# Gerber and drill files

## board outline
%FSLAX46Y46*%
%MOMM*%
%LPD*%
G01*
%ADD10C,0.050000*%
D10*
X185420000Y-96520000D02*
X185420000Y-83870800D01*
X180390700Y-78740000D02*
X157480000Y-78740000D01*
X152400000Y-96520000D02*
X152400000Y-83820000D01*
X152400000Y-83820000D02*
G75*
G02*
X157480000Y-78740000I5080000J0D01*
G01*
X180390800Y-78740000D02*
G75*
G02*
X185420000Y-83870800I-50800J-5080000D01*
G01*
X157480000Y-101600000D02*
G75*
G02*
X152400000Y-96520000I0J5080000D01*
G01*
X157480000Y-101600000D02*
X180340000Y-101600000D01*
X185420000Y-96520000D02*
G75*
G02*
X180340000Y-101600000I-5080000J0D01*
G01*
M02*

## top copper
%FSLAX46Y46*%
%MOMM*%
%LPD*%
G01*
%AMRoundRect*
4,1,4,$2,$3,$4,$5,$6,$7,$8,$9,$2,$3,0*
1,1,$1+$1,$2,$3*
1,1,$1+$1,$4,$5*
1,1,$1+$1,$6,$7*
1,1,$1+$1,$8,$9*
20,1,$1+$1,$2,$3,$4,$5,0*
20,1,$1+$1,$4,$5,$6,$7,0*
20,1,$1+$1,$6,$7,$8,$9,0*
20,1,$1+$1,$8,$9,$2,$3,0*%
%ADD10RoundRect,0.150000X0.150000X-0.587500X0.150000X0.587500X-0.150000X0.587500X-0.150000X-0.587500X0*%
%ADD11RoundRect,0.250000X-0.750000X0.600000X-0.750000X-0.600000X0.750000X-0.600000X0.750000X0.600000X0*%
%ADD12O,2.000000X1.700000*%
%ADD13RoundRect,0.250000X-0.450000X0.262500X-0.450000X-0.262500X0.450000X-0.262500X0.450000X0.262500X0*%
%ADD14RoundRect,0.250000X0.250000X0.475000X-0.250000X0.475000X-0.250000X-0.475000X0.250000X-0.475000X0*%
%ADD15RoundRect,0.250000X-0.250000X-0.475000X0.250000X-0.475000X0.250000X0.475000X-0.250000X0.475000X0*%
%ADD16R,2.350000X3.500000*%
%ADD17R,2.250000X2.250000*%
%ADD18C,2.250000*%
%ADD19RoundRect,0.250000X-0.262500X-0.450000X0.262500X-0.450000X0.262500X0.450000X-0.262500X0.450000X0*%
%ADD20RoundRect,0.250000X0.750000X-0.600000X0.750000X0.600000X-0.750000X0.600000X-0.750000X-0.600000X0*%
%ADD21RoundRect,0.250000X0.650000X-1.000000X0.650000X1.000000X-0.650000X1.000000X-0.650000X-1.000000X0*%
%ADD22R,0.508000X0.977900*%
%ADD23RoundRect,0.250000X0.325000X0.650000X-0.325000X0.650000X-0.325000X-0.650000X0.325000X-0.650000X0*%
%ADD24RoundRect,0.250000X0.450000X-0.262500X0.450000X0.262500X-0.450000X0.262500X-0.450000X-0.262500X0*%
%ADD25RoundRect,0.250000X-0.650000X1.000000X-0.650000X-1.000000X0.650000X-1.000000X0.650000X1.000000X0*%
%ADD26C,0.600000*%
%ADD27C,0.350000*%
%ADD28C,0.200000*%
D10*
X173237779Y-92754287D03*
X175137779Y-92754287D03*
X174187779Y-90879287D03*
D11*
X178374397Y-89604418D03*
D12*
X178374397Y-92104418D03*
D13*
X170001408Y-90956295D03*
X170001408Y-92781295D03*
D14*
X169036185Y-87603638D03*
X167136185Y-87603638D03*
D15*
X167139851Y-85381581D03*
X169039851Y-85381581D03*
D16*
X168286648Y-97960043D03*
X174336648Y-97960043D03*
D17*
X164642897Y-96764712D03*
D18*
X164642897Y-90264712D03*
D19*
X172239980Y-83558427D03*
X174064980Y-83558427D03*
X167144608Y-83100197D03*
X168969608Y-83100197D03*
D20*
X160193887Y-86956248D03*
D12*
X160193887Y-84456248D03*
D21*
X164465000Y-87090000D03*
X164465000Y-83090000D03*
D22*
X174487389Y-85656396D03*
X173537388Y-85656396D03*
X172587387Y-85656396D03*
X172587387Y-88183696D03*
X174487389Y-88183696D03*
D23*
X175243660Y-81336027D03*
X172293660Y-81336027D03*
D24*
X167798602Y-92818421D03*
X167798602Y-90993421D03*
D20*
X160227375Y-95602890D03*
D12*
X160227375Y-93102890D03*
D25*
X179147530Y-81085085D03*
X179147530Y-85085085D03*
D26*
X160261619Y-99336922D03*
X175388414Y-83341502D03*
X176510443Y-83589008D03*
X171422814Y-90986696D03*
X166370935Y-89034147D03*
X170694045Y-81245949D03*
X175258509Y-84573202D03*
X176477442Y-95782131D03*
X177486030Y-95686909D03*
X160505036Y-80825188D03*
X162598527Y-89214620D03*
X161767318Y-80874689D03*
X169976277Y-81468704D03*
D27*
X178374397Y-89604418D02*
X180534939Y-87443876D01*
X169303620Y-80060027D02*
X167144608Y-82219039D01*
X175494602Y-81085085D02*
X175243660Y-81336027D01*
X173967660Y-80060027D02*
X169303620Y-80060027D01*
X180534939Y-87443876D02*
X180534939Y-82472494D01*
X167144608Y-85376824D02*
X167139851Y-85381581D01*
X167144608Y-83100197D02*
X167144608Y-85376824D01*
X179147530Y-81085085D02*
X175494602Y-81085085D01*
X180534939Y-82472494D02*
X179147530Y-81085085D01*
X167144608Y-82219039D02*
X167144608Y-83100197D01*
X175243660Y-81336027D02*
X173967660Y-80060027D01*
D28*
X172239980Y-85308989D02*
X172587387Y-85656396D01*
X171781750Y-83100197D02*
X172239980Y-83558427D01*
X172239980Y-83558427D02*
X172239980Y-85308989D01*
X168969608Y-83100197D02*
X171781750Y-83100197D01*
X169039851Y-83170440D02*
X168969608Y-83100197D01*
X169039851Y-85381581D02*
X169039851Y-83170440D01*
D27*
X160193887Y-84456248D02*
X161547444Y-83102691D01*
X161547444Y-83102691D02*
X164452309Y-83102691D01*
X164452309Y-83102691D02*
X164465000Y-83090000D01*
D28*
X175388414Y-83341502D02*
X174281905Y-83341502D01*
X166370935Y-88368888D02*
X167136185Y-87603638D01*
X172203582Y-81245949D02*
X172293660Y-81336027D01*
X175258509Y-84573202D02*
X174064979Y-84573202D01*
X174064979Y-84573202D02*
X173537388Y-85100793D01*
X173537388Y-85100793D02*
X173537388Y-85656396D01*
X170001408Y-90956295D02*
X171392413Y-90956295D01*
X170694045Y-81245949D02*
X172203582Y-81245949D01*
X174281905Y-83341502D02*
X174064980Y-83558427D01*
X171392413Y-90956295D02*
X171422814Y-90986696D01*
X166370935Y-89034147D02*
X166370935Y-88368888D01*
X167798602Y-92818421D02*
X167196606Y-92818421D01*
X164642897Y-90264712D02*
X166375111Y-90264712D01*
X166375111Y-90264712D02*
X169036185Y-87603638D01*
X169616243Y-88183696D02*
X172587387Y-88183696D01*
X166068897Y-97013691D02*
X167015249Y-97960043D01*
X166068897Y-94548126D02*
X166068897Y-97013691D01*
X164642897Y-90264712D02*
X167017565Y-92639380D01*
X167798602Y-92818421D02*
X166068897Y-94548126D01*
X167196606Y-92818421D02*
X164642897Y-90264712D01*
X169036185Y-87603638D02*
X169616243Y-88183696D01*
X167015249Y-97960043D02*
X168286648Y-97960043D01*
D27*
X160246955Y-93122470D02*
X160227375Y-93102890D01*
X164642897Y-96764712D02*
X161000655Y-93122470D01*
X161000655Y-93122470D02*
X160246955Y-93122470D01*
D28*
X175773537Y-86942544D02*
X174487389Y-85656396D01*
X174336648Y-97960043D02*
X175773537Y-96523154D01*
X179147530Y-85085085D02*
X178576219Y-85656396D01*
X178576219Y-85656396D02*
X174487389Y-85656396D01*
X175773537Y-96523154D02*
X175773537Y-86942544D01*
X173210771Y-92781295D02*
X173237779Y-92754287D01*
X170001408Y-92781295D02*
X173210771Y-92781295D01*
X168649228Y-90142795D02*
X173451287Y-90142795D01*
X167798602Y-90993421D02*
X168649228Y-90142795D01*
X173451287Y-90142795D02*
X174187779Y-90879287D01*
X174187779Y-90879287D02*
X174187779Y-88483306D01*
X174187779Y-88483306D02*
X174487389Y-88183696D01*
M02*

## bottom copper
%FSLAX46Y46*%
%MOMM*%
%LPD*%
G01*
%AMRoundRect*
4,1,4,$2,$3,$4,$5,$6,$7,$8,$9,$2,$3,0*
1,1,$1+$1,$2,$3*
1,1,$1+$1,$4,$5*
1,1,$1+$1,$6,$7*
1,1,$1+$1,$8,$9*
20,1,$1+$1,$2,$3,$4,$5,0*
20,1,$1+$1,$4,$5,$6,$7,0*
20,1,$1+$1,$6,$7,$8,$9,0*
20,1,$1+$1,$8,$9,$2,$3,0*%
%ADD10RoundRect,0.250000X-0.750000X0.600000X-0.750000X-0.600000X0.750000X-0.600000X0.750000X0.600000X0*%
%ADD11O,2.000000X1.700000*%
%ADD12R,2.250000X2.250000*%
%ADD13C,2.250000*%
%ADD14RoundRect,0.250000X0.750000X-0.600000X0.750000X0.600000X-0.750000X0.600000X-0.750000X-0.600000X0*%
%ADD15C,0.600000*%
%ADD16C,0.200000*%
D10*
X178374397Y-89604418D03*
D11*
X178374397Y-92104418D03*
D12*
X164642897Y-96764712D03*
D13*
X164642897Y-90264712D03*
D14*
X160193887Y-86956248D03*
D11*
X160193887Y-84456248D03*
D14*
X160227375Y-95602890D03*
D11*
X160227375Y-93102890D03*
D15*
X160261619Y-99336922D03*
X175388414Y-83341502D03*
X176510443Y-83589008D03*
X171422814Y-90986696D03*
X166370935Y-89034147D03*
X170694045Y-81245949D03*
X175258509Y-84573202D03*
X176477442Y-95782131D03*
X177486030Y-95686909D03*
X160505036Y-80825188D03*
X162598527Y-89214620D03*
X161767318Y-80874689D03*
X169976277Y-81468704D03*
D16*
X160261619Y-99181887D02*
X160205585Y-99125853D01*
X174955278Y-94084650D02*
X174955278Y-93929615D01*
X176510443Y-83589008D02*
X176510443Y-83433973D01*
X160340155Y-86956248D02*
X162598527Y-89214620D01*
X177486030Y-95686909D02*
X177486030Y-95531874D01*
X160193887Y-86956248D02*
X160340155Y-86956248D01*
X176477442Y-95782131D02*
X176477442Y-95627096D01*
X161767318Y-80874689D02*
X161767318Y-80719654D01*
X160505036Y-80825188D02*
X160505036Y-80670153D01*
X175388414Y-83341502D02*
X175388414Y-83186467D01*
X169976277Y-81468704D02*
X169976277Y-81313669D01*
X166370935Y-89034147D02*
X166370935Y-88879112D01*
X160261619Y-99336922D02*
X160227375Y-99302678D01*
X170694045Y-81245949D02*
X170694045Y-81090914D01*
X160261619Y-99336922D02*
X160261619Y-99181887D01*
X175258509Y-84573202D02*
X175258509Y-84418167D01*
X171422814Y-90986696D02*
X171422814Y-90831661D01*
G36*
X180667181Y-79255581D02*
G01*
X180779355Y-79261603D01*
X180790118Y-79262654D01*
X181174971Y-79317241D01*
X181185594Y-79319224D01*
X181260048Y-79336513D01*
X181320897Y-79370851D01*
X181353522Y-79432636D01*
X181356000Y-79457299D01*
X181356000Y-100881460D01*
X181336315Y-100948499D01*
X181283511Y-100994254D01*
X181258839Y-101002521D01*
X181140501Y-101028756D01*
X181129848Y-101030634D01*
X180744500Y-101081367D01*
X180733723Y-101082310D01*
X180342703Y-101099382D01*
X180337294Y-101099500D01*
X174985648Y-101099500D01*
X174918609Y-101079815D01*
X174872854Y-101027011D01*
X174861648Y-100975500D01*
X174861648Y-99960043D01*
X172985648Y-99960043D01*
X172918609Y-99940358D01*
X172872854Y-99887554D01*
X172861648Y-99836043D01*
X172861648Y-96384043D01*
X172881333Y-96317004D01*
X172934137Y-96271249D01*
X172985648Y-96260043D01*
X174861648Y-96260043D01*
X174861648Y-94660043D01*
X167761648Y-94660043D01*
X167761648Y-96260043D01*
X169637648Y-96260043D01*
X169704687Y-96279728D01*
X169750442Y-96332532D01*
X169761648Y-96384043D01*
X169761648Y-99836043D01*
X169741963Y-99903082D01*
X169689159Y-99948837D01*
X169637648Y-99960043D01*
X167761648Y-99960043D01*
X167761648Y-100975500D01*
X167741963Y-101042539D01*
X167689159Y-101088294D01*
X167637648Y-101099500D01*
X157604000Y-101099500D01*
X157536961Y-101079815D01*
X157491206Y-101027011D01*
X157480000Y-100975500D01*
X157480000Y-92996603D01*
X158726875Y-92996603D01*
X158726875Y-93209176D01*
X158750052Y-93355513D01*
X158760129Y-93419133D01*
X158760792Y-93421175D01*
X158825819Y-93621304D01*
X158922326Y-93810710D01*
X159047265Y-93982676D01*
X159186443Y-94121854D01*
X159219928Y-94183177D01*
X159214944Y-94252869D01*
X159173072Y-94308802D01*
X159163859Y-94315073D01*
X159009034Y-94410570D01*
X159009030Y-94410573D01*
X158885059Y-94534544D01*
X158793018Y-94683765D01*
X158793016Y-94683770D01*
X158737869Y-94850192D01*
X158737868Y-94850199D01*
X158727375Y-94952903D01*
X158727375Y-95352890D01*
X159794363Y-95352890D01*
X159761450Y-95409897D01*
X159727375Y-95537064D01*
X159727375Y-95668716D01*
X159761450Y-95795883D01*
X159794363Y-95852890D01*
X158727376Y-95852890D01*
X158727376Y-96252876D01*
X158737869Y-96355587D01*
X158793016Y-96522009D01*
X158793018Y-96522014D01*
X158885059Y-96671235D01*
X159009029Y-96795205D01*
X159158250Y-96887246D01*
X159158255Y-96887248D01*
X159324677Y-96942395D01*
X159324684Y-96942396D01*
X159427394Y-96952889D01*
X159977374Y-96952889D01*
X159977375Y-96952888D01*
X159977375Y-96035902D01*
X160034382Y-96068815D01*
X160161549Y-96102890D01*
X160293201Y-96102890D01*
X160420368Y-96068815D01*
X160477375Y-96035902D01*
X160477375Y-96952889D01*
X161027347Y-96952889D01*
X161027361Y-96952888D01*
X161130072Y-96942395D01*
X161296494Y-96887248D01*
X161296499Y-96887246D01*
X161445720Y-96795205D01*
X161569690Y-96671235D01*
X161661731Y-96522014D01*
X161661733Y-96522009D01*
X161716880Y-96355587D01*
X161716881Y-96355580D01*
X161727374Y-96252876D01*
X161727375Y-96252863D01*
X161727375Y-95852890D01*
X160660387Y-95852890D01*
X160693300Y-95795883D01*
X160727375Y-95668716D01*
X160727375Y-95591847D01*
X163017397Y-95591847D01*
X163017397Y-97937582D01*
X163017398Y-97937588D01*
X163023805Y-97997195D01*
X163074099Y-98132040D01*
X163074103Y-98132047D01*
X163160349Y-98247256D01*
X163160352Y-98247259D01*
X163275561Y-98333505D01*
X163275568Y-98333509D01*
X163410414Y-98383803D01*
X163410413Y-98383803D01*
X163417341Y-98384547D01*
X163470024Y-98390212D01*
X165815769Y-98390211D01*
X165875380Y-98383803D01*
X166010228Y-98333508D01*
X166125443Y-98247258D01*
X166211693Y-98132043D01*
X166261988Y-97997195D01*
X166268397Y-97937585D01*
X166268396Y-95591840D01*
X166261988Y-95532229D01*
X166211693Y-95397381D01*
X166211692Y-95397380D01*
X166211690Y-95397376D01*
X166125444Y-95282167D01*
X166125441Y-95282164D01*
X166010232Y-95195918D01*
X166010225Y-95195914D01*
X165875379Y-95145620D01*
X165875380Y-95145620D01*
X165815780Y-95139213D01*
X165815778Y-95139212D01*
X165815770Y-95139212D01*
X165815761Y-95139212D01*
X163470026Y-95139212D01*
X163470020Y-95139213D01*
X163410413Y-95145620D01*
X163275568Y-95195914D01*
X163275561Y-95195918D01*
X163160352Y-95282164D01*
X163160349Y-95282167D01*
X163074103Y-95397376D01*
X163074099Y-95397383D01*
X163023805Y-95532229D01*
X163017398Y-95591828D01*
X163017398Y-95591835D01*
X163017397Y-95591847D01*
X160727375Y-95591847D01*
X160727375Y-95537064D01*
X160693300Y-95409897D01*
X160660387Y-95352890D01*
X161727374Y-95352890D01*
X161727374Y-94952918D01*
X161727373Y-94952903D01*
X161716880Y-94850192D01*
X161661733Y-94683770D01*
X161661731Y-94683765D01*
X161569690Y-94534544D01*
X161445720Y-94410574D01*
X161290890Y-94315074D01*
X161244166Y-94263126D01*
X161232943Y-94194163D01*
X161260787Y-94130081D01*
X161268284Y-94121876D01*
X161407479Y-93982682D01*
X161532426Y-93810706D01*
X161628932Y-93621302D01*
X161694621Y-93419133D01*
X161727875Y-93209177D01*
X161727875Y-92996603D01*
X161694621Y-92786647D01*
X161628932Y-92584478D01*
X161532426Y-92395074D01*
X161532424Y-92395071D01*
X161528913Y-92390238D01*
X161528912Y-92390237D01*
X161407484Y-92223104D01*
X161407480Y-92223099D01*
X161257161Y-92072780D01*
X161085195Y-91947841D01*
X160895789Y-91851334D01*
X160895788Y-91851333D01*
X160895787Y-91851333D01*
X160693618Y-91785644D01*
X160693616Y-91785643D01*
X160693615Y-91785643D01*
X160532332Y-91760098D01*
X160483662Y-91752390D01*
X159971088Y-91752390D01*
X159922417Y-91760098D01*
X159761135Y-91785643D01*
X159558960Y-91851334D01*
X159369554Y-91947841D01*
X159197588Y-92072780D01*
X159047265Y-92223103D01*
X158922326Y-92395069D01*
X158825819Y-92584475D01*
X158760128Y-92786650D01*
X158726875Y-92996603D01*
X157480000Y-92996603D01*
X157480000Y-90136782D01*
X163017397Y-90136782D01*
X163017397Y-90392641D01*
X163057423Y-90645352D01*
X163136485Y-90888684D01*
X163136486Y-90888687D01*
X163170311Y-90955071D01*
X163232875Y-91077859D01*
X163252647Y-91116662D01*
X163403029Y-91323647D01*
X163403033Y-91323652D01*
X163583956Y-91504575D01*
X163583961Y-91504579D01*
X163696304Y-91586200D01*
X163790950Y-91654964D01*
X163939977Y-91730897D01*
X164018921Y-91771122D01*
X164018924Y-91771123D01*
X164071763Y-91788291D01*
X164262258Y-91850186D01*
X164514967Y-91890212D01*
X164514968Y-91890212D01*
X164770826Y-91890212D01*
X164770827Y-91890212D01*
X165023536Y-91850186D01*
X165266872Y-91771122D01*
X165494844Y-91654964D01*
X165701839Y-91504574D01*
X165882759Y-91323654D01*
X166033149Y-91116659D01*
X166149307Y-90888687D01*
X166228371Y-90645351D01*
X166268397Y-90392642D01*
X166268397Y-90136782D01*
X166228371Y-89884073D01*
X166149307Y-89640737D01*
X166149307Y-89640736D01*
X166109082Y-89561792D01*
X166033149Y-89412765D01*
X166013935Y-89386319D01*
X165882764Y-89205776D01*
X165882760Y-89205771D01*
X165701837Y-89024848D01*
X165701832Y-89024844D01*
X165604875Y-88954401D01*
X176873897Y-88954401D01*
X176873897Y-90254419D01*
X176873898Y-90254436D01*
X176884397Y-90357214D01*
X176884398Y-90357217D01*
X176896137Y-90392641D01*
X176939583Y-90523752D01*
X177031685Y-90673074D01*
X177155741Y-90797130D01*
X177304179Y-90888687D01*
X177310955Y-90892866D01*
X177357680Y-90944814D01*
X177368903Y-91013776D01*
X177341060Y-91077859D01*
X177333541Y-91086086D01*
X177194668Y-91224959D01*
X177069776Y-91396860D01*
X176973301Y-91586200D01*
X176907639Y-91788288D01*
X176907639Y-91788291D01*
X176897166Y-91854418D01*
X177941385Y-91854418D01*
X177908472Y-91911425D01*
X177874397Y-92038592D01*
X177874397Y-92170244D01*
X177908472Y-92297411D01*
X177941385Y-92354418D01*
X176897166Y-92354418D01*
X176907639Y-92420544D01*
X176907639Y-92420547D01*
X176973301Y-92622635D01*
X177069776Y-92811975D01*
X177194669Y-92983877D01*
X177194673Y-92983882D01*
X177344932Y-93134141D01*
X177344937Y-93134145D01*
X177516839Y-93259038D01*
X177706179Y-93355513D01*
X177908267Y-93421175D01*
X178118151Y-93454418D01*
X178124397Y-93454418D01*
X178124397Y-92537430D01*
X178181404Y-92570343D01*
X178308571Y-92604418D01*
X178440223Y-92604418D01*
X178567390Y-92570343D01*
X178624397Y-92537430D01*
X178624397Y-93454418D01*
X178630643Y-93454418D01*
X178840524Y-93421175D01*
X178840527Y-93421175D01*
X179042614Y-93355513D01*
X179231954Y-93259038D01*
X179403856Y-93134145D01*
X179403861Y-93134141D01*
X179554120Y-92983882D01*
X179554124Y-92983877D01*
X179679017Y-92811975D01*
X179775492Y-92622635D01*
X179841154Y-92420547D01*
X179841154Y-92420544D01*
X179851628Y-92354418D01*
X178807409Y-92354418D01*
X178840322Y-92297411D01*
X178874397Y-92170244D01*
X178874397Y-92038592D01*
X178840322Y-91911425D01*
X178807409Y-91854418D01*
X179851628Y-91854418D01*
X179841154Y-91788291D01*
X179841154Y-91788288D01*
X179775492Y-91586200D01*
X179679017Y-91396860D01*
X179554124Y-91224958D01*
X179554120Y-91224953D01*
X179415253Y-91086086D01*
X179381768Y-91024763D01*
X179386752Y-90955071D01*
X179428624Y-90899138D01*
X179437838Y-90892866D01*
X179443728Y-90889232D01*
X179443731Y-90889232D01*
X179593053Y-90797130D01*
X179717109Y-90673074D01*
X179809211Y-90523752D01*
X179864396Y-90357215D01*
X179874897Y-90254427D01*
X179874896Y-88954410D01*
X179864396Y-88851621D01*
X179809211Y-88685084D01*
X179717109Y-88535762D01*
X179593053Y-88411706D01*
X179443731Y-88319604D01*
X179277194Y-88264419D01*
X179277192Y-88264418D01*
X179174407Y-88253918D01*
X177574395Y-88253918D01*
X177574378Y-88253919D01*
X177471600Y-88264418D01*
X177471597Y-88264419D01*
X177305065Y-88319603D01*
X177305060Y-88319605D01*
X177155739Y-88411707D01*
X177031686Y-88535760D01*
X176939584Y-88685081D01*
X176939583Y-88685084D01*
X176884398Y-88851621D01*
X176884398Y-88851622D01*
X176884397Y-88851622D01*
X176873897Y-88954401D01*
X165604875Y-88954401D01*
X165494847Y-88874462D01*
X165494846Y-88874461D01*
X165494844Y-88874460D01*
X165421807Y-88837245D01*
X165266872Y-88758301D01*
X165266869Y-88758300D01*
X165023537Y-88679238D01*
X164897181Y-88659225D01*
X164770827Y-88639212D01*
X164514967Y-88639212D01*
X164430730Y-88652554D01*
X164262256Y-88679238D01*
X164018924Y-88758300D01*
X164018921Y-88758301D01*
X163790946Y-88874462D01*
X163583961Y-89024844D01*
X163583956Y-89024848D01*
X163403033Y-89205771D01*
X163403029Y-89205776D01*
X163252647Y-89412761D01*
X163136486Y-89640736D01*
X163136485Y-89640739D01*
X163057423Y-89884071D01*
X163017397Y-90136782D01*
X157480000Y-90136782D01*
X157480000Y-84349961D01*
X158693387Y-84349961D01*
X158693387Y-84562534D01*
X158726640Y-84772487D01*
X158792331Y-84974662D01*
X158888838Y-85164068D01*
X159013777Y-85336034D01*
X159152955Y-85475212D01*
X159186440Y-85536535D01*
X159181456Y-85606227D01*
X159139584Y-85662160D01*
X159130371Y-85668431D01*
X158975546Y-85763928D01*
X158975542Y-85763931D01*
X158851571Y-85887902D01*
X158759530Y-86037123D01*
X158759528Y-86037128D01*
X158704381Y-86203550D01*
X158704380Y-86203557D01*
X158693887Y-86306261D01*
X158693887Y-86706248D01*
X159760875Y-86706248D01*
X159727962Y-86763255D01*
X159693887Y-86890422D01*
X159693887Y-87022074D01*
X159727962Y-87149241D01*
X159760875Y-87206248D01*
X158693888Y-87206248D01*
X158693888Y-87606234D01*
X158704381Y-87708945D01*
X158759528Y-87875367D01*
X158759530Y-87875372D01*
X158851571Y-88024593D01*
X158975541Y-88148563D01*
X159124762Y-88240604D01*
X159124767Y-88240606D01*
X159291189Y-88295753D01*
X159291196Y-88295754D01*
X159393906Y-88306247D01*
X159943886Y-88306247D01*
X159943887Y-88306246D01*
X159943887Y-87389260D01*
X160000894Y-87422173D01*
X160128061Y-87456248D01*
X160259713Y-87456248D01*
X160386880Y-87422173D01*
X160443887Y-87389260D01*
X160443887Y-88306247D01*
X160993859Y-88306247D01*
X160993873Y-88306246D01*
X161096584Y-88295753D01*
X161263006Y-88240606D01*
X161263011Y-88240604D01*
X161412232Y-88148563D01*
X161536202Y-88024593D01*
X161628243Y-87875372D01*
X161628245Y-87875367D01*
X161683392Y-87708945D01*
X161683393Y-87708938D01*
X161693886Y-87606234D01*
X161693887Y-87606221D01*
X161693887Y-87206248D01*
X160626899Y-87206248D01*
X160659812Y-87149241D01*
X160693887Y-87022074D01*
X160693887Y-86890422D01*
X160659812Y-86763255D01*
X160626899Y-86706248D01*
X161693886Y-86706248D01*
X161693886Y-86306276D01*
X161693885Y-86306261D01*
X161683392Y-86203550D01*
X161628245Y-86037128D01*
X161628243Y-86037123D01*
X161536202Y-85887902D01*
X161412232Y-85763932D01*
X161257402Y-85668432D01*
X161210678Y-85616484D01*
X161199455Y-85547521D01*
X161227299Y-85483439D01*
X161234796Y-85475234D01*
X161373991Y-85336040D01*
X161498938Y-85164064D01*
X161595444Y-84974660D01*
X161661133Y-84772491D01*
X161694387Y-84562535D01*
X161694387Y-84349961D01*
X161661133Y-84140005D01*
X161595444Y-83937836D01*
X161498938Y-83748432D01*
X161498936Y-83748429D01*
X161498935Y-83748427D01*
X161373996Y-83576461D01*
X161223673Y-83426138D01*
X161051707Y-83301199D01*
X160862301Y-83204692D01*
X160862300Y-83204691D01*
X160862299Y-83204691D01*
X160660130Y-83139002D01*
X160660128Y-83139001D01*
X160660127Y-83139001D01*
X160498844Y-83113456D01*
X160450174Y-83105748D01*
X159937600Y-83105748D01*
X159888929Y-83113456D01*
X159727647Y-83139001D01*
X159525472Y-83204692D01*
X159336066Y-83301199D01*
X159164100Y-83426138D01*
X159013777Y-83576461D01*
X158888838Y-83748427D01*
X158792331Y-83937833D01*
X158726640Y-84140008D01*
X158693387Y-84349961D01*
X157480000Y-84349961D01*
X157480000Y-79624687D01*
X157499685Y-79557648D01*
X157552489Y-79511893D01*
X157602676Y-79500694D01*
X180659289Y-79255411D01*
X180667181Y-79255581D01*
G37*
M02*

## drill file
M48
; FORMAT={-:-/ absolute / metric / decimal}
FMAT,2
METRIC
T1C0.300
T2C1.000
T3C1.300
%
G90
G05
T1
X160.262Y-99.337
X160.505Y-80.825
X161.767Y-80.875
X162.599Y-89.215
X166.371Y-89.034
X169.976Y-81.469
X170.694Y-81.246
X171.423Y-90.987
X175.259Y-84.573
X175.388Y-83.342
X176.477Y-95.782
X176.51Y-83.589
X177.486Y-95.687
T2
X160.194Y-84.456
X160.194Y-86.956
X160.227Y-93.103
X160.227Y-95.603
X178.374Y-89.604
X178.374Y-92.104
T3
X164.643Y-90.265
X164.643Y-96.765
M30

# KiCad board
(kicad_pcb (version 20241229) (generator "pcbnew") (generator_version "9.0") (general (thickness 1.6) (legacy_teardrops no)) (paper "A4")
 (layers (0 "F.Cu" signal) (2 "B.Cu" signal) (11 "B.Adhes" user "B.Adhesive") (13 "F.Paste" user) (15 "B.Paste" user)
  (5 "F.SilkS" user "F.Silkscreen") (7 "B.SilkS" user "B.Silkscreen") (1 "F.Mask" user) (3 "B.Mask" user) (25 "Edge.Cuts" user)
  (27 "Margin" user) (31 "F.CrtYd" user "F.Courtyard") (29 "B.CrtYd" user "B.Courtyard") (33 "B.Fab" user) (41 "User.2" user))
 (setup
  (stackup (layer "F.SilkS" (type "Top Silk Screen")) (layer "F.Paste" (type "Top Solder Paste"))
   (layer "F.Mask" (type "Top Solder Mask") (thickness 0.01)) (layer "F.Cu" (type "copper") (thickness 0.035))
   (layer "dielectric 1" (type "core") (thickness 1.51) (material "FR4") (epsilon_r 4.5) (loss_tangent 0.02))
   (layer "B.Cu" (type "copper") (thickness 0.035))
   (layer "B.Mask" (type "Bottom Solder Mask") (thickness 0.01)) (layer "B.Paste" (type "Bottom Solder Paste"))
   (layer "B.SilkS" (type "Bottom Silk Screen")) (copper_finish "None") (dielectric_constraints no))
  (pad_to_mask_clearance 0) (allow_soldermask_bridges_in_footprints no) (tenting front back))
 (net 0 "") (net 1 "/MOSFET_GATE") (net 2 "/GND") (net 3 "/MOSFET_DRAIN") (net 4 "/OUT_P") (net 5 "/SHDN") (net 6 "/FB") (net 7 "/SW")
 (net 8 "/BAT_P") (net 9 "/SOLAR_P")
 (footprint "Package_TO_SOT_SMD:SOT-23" (layer "F.Cu") (at 174.187779 91.816787 90)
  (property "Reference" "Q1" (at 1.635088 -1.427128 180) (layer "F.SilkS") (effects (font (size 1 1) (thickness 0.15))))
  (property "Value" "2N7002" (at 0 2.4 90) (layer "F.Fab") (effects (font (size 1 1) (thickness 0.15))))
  (pad "1" smd roundrect (at -0.9375 -0.95 90) (size 1.475 0.6) (layers "F.Cu" "F.Mask" "F.Paste") (roundrect_rratio 0.25)
   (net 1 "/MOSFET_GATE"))
  (pad "2" smd roundrect (at -0.9375 0.95 90) (size 1.475 0.6) (layers "F.Cu" "F.Mask" "F.Paste") (roundrect_rratio 0.25) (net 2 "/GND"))
  (pad "3" smd roundrect (at 0.9375 0 90) (size 1.475 0.6) (layers "F.Cu" "F.Mask" "F.Paste") (roundrect_rratio 0.25)
   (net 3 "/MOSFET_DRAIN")))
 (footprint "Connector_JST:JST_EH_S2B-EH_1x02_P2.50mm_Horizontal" (layer "F.Cu") (at 178.374397 89.604418 -90)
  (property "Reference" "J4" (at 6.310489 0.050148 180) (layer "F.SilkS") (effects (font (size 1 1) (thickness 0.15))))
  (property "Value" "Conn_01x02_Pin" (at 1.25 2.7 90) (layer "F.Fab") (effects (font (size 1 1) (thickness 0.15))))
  (pad "1" thru_hole roundrect (at 0 0 270) (size 1.7 2) (drill 1) (layers "*.Cu" "*.Mask") (remove_unused_layers no)
   (roundrect_rratio 0.147059) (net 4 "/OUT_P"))
  (pad "2" thru_hole oval (at 2.5 0 270) (size 1.7 2) (drill 1) (layers "*.Cu" "*.Mask") (remove_unused_layers no) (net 2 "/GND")))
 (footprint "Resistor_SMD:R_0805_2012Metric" (layer "F.Cu") (at 170.001408 91.868795 -90)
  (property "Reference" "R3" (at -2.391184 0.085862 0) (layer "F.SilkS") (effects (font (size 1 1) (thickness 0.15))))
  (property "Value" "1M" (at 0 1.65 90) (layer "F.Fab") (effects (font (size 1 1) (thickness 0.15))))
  (pad "1" smd roundrect (at -0.9125 0 270) (size 1.025 1.4) (layers "F.Cu" "F.Mask" "F.Paste") (roundrect_rratio 0.243902) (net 2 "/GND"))
  (pad "2" smd roundrect (at 0.9125 0 270) (size 1.025 1.4) (layers "F.Cu" "F.Mask" "F.Paste") (roundrect_rratio 0.243902)
   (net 1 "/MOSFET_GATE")))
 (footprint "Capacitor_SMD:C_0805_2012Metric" (layer "F.Cu") (at 168.086185 87.603638 180)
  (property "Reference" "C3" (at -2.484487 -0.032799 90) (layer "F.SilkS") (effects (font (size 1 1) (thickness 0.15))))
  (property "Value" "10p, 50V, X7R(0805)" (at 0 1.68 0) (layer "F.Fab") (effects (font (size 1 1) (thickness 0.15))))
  (pad "1" smd roundrect (at -0.95 0 180) (size 1 1.45) (layers "F.Cu" "F.Mask" "F.Paste") (roundrect_rratio 0.25) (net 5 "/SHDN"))
  (pad "2" smd roundrect (at 0.95 0 180) (size 1 1.45) (layers "F.Cu" "F.Mask" "F.Paste") (roundrect_rratio 0.25) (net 2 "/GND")))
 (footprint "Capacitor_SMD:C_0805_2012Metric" (layer "F.Cu") (at 168.089851 85.381581)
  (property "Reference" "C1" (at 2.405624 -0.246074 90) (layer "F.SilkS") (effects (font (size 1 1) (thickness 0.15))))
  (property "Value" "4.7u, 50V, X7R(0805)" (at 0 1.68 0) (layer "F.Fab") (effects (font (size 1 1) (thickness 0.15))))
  (pad "1" smd roundrect (at -0.95 0) (size 1 1.45) (layers "F.Cu" "F.Mask" "F.Paste") (roundrect_rratio 0.25) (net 4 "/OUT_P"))
  (pad "2" smd roundrect (at 0.95 0) (size 1 1.45) (layers "F.Cu" "F.Mask" "F.Paste") (roundrect_rratio 0.25) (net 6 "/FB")))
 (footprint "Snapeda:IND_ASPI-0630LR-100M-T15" (layer "F.Cu") (at 171.311648 97.960043)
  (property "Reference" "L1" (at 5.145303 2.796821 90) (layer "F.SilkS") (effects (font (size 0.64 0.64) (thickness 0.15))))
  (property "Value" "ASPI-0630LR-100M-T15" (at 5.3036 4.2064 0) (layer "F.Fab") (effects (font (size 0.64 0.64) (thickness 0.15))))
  (pad "1" smd rect (at -3.025 0) (size 2.35 3.5) (layers "F.Cu" "F.Mask" "F.Paste") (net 5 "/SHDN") (solder_mask_margin 0.102))
  (pad "2" smd rect (at 3.025 0) (size 2.35 3.5) (layers "F.Cu" "F.Mask" "F.Paste") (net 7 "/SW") (solder_mask_margin 0.102))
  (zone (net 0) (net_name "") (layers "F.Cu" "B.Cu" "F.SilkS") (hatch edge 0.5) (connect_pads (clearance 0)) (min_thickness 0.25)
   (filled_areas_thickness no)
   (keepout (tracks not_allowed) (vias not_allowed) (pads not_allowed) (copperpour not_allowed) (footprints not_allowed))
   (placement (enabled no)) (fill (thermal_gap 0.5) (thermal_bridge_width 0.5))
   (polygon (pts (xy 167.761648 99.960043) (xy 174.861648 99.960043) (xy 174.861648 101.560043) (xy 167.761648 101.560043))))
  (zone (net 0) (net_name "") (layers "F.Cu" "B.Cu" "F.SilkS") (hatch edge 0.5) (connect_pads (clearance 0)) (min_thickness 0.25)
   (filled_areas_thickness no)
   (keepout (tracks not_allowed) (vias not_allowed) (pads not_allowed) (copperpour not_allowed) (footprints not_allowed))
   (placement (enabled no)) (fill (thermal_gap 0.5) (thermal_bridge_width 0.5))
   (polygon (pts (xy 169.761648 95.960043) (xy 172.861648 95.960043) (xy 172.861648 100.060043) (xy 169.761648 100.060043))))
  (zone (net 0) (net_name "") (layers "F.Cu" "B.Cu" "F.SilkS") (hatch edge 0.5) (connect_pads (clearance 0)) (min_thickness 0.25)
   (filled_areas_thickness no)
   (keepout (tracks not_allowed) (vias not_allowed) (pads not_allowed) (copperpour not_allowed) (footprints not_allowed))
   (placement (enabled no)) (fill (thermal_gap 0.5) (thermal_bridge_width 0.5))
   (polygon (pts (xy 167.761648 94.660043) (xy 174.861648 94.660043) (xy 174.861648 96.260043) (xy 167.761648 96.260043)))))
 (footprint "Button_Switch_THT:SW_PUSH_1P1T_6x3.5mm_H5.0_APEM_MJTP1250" (layer "F.Cu") (at 164.642897 96.764712 90)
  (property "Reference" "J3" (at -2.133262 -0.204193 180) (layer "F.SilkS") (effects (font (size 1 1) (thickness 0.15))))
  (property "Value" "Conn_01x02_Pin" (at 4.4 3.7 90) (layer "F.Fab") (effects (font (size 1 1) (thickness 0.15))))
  (pad "1" thru_hole rect (at 0 0 180) (size 2.25 2.25) (drill 1.3) (layers "*.Cu" "*.Mask") (remove_unused_layers no) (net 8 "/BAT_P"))
  (pad "2" thru_hole circle (at 6.5 0 180) (size 2.25 2.25) (drill 1.3) (layers "*.Cu" "*.Mask") (remove_unused_layers no) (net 5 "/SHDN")))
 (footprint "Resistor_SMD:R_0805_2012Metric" (layer "F.Cu") (at 173.15248 83.558427)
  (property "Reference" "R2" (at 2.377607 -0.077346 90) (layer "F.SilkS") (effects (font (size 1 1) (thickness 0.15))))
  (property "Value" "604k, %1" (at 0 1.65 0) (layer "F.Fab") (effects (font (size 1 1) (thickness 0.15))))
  (pad "1" smd roundrect (at -0.9125 0) (size 1.025 1.4) (layers "F.Cu" "F.Mask" "F.Paste") (roundrect_rratio 0.243902) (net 6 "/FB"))
  (pad "2" smd roundrect (at 0.9125 0) (size 1.025 1.4) (layers "F.Cu" "F.Mask" "F.Paste") (roundrect_rratio 0.243902) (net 2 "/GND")))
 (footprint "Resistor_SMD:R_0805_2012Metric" (layer "F.Cu") (at 168.057108 83.100197)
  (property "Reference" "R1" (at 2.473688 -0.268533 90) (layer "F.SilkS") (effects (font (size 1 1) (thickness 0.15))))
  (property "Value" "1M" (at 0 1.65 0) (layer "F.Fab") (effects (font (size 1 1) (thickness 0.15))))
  (pad "1" smd roundrect (at -0.9125 0) (size 1.025 1.4) (layers "F.Cu" "F.Mask" "F.Paste") (roundrect_rratio 0.243902) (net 4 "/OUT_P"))
  (pad "2" smd roundrect (at 0.9125 0) (size 1.025 1.4) (layers "F.Cu" "F.Mask" "F.Paste") (roundrect_rratio 0.243902) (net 6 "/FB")))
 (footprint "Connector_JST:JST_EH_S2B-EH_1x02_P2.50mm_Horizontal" (layer "F.Cu") (at 160.193887 86.956248 90)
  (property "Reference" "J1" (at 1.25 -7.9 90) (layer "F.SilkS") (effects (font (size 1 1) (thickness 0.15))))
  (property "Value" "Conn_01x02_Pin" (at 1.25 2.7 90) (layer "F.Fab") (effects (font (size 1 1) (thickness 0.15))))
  (pad "1" thru_hole roundrect (at 0 0 90) (size 1.7 2) (drill 1) (layers "*.Cu" "*.Mask") (remove_unused_layers no)
   (roundrect_rratio 0.147059) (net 2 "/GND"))
  (pad "2" thru_hole oval (at 2.5 0 90) (size 1.7 2) (drill 1) (layers "*.Cu" "*.Mask") (remove_unused_layers no) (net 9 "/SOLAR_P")))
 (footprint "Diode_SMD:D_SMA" (layer "F.Cu") (at 164.465 85.09 90)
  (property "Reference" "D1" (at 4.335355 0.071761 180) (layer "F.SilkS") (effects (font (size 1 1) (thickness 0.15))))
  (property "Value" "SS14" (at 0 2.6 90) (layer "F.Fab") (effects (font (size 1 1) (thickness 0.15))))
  (pad "1" smd roundrect (at -2 0 90) (size 2.5 1.8) (layers "F.Cu" "F.Mask" "F.Paste") (roundrect_rratio 0.1388888889) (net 8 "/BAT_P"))
  (pad "2" smd roundrect (at 2 0 90) (size 2.5 1.8) (layers "F.Cu" "F.Mask" "F.Paste") (roundrect_rratio 0.1388888889) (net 9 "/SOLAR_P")))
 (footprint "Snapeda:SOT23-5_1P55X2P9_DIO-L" (layer "F.Cu") (at 173.537388 86.920046 -90)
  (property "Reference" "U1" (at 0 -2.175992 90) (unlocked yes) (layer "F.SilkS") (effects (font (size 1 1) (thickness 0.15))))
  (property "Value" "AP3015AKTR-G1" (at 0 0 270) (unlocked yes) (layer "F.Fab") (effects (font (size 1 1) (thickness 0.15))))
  (pad "1" smd rect (at -1.26365 -0.950001 270) (size 0.9779 0.508) (layers "F.Cu" "F.Mask" "F.Paste") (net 7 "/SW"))
  (pad "2" smd rect (at -1.26365 0 270) (size 0.9779 0.508) (layers "F.Cu" "F.Mask" "F.Paste") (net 2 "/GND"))
  (pad "3" smd rect (at -1.26365 0.950001 270) (size 0.9779 0.508) (layers "F.Cu" "F.Mask" "F.Paste") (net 6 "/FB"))
  (pad "4" smd rect (at 1.26365 0.950001 270) (size 0.9779 0.508) (layers "F.Cu" "F.Mask" "F.Paste") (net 5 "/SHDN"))
  (pad "5" smd rect (at 1.26365 -0.950001 270) (size 0.9779 0.508) (layers "F.Cu" "F.Mask" "F.Paste") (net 3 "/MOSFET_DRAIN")))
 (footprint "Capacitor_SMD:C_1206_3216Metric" (layer "F.Cu") (at 173.76866 81.336027 180)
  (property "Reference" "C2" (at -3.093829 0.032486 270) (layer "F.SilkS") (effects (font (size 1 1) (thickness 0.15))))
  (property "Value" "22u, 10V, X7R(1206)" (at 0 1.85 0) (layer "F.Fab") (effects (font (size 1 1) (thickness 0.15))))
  (pad "1" smd roundrect (at -1.475 0 180) (size 1.15 1.8) (layers "F.Cu" "F.Mask" "F.Paste") (roundrect_rratio 0.217391) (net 4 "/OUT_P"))
  (pad "2" smd roundrect (at 1.475 0 180) (size 1.15 1.8) (layers "F.Cu" "F.Mask" "F.Paste") (roundrect_rratio 0.217391) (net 2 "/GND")))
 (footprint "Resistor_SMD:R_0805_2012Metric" (layer "F.Cu") (at 167.798602 91.905921 90)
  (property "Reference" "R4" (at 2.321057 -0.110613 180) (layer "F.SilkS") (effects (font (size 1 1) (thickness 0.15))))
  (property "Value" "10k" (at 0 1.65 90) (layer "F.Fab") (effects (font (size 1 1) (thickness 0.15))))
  (pad "1" smd roundrect (at -0.9125 0 90) (size 1.025 1.4) (layers "F.Cu" "F.Mask" "F.Paste") (roundrect_rratio 0.243902) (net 5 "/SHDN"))
  (pad "2" smd roundrect (at 0.9125 0 90) (size 1.025 1.4) (layers "F.Cu" "F.Mask" "F.Paste") (roundrect_rratio 0.243902)
   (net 3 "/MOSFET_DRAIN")))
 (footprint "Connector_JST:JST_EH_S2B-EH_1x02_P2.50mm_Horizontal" (layer "F.Cu") (at 160.227375 95.60289 90)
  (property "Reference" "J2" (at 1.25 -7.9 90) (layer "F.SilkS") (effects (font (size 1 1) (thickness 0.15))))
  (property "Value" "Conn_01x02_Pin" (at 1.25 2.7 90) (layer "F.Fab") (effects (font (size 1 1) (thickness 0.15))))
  (pad "1" thru_hole roundrect (at 0 0 90) (size 1.7 2) (drill 1) (layers "*.Cu" "*.Mask") (remove_unused_layers no)
   (roundrect_rratio 0.147059) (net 2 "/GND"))
  (pad "2" thru_hole oval (at 2.5 0 90) (size 1.7 2) (drill 1) (layers "*.Cu" "*.Mask") (remove_unused_layers no) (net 8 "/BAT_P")))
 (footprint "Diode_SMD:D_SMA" (layer "F.Cu") (at 179.14753 83.085085 -90)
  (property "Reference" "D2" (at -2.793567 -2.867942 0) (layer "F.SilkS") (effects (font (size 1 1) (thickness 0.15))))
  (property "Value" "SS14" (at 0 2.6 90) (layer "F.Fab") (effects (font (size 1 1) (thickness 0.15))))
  (pad "1" smd roundrect (at -2 0 270) (size 2.5 1.8) (layers "F.Cu" "F.Mask" "F.Paste") (roundrect_rratio 0.1388888889) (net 4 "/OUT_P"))
  (pad "2" smd roundrect (at 2 0 270) (size 2.5 1.8) (layers "F.Cu" "F.Mask" "F.Paste") (roundrect_rratio 0.1388888889) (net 7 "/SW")))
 (gr_line (start 185.42 96.52) (end 185.42 83.8708) (stroke (width 0.05) (type default)) (layer "Edge.Cuts"))
 (gr_line (start 180.3907 78.74) (end 157.48 78.74) (stroke (width 0.05) (type default)) (layer "Edge.Cuts"))
 (gr_line (start 152.4 96.52) (end 152.4 83.82) (stroke (width 0.05) (type default)) (layer "Edge.Cuts"))
 (gr_arc (start 152.4 83.82) (mid 153.887898 80.227898) (end 157.48 78.74) (stroke (width 0.05) (type default)) (layer "Edge.Cuts"))
 (gr_arc (start 180.3908 78.74) (mid 183.968023 80.263819) (end 185.42 83.8708) (stroke (width 0.05) (type default)) (layer "Edge.Cuts"))
 (gr_arc (start 157.48 101.6) (mid 153.887898 100.112102) (end 152.4 96.52) (stroke (width 0.05) (type default)) (layer "Edge.Cuts"))
 (gr_line (start 157.48 101.6) (end 180.34 101.6) (stroke (width 0.05) (type default)) (layer "Edge.Cuts"))
 (gr_arc (start 185.42 96.52) (mid 183.932102 100.112102) (end 180.34 101.6) (stroke (width 0.05) (type default)) (layer "Edge.Cuts"))
 (segment (start 178.374397 89.604418) (end 180.534939 87.443876) (width 0.35) (layer "F.Cu") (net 4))
 (segment (start 169.30362 80.060027) (end 167.144608 82.219039) (width 0.35) (layer "F.Cu") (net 4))
 (segment (start 175.494602 81.085085) (end 175.24366 81.336027) (width 0.35) (layer "F.Cu") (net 4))
 (segment (start 173.96766 80.060027) (end 169.30362 80.060027) (width 0.35) (layer "F.Cu") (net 4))
 (segment (start 180.534939 87.443876) (end 180.534939 82.472494) (width 0.35) (layer "F.Cu") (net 4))
 (segment (start 167.144608 85.376824) (end 167.139851 85.381581) (width 0.35) (layer "F.Cu") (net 4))
 (segment (start 167.144608 83.100197) (end 167.144608 85.376824) (width 0.35) (layer "F.Cu") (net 4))
 (segment (start 179.14753 81.085085) (end 175.494602 81.085085) (width 0.35) (layer "F.Cu") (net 4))
 (segment (start 180.534939 82.472494) (end 179.14753 81.085085) (width 0.35) (layer "F.Cu") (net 4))
 (segment (start 167.144608 82.219039) (end 167.144608 83.100197) (width 0.35) (layer "F.Cu") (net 4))
 (segment (start 175.24366 81.336027) (end 173.96766 80.060027) (width 0.35) (layer "F.Cu") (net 4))
 (segment (start 172.23998 85.308989) (end 172.587387 85.656396) (width 0.2) (layer "F.Cu") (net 6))
 (segment (start 171.78175 83.100197) (end 172.23998 83.558427) (width 0.2) (layer "F.Cu") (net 6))
 (segment (start 172.23998 83.558427) (end 172.23998 85.308989) (width 0.2) (layer "F.Cu") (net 6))
 (segment (start 168.969608 83.100197) (end 171.78175 83.100197) (width 0.2) (layer "F.Cu") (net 6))
 (segment (start 169.039851 83.17044) (end 168.969608 83.100197) (width 0.2) (layer "F.Cu") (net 6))
 (segment (start 169.039851 85.381581) (end 169.039851 83.17044) (width 0.2) (layer "F.Cu") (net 6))
 (segment (start 160.193887 84.456248) (end 161.547444 83.102691) (width 0.35) (layer "F.Cu") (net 9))
 (segment (start 161.547444 83.102691) (end 164.452309 83.102691) (width 0.35) (layer "F.Cu") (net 9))
 (segment (start 164.452309 83.102691) (end 164.465 83.09) (width 0.35) (layer "F.Cu") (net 9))
 (segment (start 175.388414 83.341502) (end 174.281905 83.341502) (width 0.2) (layer "F.Cu") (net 2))
 (segment (start 166.370935 88.368888) (end 167.136185 87.603638) (width 0.2) (layer "F.Cu") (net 2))
 (segment (start 172.203582 81.245949) (end 172.29366 81.336027) (width 0.2) (layer "F.Cu") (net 2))
 (segment (start 175.258509 84.573202) (end 174.064979 84.573202) (width 0.2) (layer "F.Cu") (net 2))
 (segment (start 174.064979 84.573202) (end 173.537388 85.100793) (width 0.2) (layer "F.Cu") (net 2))
 (segment (start 173.537388 85.100793) (end 173.537388 85.656396) (width 0.2) (layer "F.Cu") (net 2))
 (segment (start 170.001408 90.956295) (end 171.392413 90.956295) (width 0.2) (layer "F.Cu") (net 2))
 (segment (start 170.694045 81.245949) (end 172.203582 81.245949) (width 0.2) (layer "F.Cu") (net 2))
 (segment (start 174.281905 83.341502) (end 174.06498 83.558427) (width 0.2) (layer "F.Cu") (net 2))
 (segment (start 171.392413 90.956295) (end 171.422814 90.986696) (width 0.2) (layer "F.Cu") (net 2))
 (segment (start 166.370935 89.034147) (end 166.370935 88.368888) (width 0.2) (layer "F.Cu") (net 2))
 (via (at 160.261619 99.336922) (size 0.6) (drill 0.3) (layers "F.Cu" "B.Cu") (free yes) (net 2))
 (via (at 175.388414 83.341502) (size 0.6) (drill 0.3) (layers "F.Cu" "B.Cu") (free yes) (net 2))
 (via (at 176.510443 83.589008) (size 0.6) (drill 0.3) (layers "F.Cu" "B.Cu") (free yes) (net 2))
 (via (at 171.422814 90.986696) (size 0.6) (drill 0.3) (layers "F.Cu" "B.Cu") (free yes) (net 2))
 (via (at 166.370935 89.034147) (size 0.6) (drill 0.3) (layers "F.Cu" "B.Cu") (free yes) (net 2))
 (via (at 170.694045 81.245949) (size 0.6) (drill 0.3) (layers "F.Cu" "B.Cu") (free yes) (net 2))
 (via (at 175.258509 84.573202) (size 0.6) (drill 0.3) (layers "F.Cu" "B.Cu") (free yes) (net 2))
 (via (at 176.477442 95.782131) (size 0.6) (drill 0.3) (layers "F.Cu" "B.Cu") (free yes) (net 2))
 (via (at 177.48603 95.686909) (size 0.6) (drill 0.3) (layers "F.Cu" "B.Cu") (free yes) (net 2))
 (via (at 160.505036 80.825188) (size 0.6) (drill 0.3) (layers "F.Cu" "B.Cu") (free yes) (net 2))
 (via (at 162.598527 89.21462) (size 0.6) (drill 0.3) (layers "F.Cu" "B.Cu") (free yes) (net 2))
 (via (at 161.767318 80.874689) (size 0.6) (drill 0.3) (layers "F.Cu" "B.Cu") (free yes) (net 2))
 (via (at 169.976277 81.468704) (size 0.6) (drill 0.3) (layers "F.Cu" "B.Cu") (free yes) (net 2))
 (segment (start 160.261619 99.181887) (end 160.205585 99.125853) (width 0.2) (layer "B.Cu") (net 2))
 (segment (start 174.955278 94.08465) (end 174.955278 93.929615) (width 0.2) (layer "B.Cu") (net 2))
 (segment (start 176.510443 83.589008) (end 176.510443 83.433973) (width 0.2) (layer "B.Cu") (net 2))
 (segment (start 160.340155 86.956248) (end 162.598527 89.21462) (width 0.2) (layer "B.Cu") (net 2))
 (segment (start 177.48603 95.686909) (end 177.48603 95.531874) (width 0.2) (layer "B.Cu") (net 2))
 (segment (start 160.193887 86.956248) (end 160.340155 86.956248) (width 0.2) (layer "B.Cu") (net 2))
 (segment (start 176.477442 95.782131) (end 176.477442 95.627096) (width 0.2) (layer "B.Cu") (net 2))
 (segment (start 161.767318 80.874689) (end 161.767318 80.719654) (width 0.2) (layer "B.Cu") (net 2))
 (segment (start 160.505036 80.825188) (end 160.505036 80.670153) (width 0.2) (layer "B.Cu") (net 2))
 (segment (start 175.388414 83.341502) (end 175.388414 83.186467) (width 0.2) (layer "B.Cu") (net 2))
 (segment (start 169.976277 81.468704) (end 169.976277 81.313669) (width 0.2) (layer "B.Cu") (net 2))
 (segment (start 166.370935 89.034147) (end 166.370935 88.879112) (width 0.2) (layer "B.Cu") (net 2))
 (segment (start 160.261619 99.336922) (end 160.227375 99.302678) (width 0.2) (layer "B.Cu") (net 2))
 (segment (start 170.694045 81.245949) (end 170.694045 81.090914) (width 0.2) (layer "B.Cu") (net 2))
 (segment (start 160.261619 99.336922) (end 160.261619 99.181887) (width 0.2) (layer "B.Cu") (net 2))
 (segment (start 175.258509 84.573202) (end 175.258509 84.418167) (width 0.2) (layer "B.Cu") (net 2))
 (segment (start 171.422814 90.986696) (end 171.422814 90.831661) (width 0.2) (layer "B.Cu") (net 2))
 (segment (start 167.798602 92.818421) (end 167.196606 92.818421) (width 0.2) (layer "F.Cu") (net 5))
 (segment (start 164.642897 90.264712) (end 166.375111 90.264712) (width 0.2) (layer "F.Cu") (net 5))
 (segment (start 166.375111 90.264712) (end 169.036185 87.603638) (width 0.2) (layer "F.Cu") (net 5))
 (segment (start 169.616243 88.183696) (end 172.587387 88.183696) (width 0.2) (layer "F.Cu") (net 5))
 (segment (start 166.068897 97.013691) (end 167.015249 97.960043) (width 0.2) (layer "F.Cu") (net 5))
 (segment (start 166.068897 94.548126) (end 166.068897 97.013691) (width 0.2) (layer "F.Cu") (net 5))
 (segment (start 164.642897 90.264712) (end 167.017565 92.63938) (width 0.2) (layer "F.Cu") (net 5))
 (segment (start 167.798602 92.818421) (end 166.068897 94.548126) (width 0.2) (layer "F.Cu") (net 5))
 (segment (start 167.196606 92.818421) (end 164.642897 90.264712) (width 0.2) (layer "F.Cu") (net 5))
 (segment (start 169.036185 87.603638) (end 169.616243 88.183696) (width 0.2) (layer "F.Cu") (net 5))
 (segment (start 167.015249 97.960043) (end 168.286648 97.960043) (width 0.2) (layer "F.Cu") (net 5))
 (segment (start 160.246955 93.12247) (end 160.227375 93.10289) (width 0.35) (layer "F.Cu") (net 8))
 (segment (start 164.642897 96.764712) (end 161.000655 93.12247) (width 0.35) (layer "F.Cu") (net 8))
 (segment (start 161.000655 93.12247) (end 160.246955 93.12247) (width 0.35) (layer "F.Cu") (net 8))
 (segment (start 175.773537 86.942544) (end 174.487389 85.656396) (width 0.2) (layer "F.Cu") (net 7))
 (segment (start 174.336648 97.960043) (end 175.773537 96.523154) (width 0.2) (layer "F.Cu") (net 7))
 (segment (start 179.14753 85.085085) (end 178.576219 85.656396) (width 0.2) (layer "F.Cu") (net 7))
 (segment (start 178.576219 85.656396) (end 174.487389 85.656396) (width 0.2) (layer "F.Cu") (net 7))
 (segment (start 175.773537 96.523154) (end 175.773537 86.942544) (width 0.2) (layer "F.Cu") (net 7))
 (segment (start 173.210771 92.781295) (end 173.237779 92.754287) (width 0.2) (layer "F.Cu") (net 1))
 (segment (start 170.001408 92.781295) (end 173.210771 92.781295) (width 0.2) (layer "F.Cu") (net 1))
 (segment (start 168.649228 90.142795) (end 173.451287 90.142795) (width 0.2) (layer "F.Cu") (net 3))
 (segment (start 167.798602 90.993421) (end 168.649228 90.142795) (width 0.2) (layer "F.Cu") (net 3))
 (segment (start 173.451287 90.142795) (end 174.187779 90.879287) (width 0.2) (layer "F.Cu") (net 3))
 (segment (start 174.187779 90.879287) (end 174.187779 88.483306) (width 0.2) (layer "F.Cu") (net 3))
 (segment (start 174.187779 88.483306) (end 174.487389 88.183696) (width 0.2) (layer "F.Cu") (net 3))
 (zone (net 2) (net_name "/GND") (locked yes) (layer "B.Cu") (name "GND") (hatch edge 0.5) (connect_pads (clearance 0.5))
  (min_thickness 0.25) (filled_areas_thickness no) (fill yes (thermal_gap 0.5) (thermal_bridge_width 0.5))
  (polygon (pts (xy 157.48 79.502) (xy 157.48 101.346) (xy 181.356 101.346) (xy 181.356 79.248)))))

